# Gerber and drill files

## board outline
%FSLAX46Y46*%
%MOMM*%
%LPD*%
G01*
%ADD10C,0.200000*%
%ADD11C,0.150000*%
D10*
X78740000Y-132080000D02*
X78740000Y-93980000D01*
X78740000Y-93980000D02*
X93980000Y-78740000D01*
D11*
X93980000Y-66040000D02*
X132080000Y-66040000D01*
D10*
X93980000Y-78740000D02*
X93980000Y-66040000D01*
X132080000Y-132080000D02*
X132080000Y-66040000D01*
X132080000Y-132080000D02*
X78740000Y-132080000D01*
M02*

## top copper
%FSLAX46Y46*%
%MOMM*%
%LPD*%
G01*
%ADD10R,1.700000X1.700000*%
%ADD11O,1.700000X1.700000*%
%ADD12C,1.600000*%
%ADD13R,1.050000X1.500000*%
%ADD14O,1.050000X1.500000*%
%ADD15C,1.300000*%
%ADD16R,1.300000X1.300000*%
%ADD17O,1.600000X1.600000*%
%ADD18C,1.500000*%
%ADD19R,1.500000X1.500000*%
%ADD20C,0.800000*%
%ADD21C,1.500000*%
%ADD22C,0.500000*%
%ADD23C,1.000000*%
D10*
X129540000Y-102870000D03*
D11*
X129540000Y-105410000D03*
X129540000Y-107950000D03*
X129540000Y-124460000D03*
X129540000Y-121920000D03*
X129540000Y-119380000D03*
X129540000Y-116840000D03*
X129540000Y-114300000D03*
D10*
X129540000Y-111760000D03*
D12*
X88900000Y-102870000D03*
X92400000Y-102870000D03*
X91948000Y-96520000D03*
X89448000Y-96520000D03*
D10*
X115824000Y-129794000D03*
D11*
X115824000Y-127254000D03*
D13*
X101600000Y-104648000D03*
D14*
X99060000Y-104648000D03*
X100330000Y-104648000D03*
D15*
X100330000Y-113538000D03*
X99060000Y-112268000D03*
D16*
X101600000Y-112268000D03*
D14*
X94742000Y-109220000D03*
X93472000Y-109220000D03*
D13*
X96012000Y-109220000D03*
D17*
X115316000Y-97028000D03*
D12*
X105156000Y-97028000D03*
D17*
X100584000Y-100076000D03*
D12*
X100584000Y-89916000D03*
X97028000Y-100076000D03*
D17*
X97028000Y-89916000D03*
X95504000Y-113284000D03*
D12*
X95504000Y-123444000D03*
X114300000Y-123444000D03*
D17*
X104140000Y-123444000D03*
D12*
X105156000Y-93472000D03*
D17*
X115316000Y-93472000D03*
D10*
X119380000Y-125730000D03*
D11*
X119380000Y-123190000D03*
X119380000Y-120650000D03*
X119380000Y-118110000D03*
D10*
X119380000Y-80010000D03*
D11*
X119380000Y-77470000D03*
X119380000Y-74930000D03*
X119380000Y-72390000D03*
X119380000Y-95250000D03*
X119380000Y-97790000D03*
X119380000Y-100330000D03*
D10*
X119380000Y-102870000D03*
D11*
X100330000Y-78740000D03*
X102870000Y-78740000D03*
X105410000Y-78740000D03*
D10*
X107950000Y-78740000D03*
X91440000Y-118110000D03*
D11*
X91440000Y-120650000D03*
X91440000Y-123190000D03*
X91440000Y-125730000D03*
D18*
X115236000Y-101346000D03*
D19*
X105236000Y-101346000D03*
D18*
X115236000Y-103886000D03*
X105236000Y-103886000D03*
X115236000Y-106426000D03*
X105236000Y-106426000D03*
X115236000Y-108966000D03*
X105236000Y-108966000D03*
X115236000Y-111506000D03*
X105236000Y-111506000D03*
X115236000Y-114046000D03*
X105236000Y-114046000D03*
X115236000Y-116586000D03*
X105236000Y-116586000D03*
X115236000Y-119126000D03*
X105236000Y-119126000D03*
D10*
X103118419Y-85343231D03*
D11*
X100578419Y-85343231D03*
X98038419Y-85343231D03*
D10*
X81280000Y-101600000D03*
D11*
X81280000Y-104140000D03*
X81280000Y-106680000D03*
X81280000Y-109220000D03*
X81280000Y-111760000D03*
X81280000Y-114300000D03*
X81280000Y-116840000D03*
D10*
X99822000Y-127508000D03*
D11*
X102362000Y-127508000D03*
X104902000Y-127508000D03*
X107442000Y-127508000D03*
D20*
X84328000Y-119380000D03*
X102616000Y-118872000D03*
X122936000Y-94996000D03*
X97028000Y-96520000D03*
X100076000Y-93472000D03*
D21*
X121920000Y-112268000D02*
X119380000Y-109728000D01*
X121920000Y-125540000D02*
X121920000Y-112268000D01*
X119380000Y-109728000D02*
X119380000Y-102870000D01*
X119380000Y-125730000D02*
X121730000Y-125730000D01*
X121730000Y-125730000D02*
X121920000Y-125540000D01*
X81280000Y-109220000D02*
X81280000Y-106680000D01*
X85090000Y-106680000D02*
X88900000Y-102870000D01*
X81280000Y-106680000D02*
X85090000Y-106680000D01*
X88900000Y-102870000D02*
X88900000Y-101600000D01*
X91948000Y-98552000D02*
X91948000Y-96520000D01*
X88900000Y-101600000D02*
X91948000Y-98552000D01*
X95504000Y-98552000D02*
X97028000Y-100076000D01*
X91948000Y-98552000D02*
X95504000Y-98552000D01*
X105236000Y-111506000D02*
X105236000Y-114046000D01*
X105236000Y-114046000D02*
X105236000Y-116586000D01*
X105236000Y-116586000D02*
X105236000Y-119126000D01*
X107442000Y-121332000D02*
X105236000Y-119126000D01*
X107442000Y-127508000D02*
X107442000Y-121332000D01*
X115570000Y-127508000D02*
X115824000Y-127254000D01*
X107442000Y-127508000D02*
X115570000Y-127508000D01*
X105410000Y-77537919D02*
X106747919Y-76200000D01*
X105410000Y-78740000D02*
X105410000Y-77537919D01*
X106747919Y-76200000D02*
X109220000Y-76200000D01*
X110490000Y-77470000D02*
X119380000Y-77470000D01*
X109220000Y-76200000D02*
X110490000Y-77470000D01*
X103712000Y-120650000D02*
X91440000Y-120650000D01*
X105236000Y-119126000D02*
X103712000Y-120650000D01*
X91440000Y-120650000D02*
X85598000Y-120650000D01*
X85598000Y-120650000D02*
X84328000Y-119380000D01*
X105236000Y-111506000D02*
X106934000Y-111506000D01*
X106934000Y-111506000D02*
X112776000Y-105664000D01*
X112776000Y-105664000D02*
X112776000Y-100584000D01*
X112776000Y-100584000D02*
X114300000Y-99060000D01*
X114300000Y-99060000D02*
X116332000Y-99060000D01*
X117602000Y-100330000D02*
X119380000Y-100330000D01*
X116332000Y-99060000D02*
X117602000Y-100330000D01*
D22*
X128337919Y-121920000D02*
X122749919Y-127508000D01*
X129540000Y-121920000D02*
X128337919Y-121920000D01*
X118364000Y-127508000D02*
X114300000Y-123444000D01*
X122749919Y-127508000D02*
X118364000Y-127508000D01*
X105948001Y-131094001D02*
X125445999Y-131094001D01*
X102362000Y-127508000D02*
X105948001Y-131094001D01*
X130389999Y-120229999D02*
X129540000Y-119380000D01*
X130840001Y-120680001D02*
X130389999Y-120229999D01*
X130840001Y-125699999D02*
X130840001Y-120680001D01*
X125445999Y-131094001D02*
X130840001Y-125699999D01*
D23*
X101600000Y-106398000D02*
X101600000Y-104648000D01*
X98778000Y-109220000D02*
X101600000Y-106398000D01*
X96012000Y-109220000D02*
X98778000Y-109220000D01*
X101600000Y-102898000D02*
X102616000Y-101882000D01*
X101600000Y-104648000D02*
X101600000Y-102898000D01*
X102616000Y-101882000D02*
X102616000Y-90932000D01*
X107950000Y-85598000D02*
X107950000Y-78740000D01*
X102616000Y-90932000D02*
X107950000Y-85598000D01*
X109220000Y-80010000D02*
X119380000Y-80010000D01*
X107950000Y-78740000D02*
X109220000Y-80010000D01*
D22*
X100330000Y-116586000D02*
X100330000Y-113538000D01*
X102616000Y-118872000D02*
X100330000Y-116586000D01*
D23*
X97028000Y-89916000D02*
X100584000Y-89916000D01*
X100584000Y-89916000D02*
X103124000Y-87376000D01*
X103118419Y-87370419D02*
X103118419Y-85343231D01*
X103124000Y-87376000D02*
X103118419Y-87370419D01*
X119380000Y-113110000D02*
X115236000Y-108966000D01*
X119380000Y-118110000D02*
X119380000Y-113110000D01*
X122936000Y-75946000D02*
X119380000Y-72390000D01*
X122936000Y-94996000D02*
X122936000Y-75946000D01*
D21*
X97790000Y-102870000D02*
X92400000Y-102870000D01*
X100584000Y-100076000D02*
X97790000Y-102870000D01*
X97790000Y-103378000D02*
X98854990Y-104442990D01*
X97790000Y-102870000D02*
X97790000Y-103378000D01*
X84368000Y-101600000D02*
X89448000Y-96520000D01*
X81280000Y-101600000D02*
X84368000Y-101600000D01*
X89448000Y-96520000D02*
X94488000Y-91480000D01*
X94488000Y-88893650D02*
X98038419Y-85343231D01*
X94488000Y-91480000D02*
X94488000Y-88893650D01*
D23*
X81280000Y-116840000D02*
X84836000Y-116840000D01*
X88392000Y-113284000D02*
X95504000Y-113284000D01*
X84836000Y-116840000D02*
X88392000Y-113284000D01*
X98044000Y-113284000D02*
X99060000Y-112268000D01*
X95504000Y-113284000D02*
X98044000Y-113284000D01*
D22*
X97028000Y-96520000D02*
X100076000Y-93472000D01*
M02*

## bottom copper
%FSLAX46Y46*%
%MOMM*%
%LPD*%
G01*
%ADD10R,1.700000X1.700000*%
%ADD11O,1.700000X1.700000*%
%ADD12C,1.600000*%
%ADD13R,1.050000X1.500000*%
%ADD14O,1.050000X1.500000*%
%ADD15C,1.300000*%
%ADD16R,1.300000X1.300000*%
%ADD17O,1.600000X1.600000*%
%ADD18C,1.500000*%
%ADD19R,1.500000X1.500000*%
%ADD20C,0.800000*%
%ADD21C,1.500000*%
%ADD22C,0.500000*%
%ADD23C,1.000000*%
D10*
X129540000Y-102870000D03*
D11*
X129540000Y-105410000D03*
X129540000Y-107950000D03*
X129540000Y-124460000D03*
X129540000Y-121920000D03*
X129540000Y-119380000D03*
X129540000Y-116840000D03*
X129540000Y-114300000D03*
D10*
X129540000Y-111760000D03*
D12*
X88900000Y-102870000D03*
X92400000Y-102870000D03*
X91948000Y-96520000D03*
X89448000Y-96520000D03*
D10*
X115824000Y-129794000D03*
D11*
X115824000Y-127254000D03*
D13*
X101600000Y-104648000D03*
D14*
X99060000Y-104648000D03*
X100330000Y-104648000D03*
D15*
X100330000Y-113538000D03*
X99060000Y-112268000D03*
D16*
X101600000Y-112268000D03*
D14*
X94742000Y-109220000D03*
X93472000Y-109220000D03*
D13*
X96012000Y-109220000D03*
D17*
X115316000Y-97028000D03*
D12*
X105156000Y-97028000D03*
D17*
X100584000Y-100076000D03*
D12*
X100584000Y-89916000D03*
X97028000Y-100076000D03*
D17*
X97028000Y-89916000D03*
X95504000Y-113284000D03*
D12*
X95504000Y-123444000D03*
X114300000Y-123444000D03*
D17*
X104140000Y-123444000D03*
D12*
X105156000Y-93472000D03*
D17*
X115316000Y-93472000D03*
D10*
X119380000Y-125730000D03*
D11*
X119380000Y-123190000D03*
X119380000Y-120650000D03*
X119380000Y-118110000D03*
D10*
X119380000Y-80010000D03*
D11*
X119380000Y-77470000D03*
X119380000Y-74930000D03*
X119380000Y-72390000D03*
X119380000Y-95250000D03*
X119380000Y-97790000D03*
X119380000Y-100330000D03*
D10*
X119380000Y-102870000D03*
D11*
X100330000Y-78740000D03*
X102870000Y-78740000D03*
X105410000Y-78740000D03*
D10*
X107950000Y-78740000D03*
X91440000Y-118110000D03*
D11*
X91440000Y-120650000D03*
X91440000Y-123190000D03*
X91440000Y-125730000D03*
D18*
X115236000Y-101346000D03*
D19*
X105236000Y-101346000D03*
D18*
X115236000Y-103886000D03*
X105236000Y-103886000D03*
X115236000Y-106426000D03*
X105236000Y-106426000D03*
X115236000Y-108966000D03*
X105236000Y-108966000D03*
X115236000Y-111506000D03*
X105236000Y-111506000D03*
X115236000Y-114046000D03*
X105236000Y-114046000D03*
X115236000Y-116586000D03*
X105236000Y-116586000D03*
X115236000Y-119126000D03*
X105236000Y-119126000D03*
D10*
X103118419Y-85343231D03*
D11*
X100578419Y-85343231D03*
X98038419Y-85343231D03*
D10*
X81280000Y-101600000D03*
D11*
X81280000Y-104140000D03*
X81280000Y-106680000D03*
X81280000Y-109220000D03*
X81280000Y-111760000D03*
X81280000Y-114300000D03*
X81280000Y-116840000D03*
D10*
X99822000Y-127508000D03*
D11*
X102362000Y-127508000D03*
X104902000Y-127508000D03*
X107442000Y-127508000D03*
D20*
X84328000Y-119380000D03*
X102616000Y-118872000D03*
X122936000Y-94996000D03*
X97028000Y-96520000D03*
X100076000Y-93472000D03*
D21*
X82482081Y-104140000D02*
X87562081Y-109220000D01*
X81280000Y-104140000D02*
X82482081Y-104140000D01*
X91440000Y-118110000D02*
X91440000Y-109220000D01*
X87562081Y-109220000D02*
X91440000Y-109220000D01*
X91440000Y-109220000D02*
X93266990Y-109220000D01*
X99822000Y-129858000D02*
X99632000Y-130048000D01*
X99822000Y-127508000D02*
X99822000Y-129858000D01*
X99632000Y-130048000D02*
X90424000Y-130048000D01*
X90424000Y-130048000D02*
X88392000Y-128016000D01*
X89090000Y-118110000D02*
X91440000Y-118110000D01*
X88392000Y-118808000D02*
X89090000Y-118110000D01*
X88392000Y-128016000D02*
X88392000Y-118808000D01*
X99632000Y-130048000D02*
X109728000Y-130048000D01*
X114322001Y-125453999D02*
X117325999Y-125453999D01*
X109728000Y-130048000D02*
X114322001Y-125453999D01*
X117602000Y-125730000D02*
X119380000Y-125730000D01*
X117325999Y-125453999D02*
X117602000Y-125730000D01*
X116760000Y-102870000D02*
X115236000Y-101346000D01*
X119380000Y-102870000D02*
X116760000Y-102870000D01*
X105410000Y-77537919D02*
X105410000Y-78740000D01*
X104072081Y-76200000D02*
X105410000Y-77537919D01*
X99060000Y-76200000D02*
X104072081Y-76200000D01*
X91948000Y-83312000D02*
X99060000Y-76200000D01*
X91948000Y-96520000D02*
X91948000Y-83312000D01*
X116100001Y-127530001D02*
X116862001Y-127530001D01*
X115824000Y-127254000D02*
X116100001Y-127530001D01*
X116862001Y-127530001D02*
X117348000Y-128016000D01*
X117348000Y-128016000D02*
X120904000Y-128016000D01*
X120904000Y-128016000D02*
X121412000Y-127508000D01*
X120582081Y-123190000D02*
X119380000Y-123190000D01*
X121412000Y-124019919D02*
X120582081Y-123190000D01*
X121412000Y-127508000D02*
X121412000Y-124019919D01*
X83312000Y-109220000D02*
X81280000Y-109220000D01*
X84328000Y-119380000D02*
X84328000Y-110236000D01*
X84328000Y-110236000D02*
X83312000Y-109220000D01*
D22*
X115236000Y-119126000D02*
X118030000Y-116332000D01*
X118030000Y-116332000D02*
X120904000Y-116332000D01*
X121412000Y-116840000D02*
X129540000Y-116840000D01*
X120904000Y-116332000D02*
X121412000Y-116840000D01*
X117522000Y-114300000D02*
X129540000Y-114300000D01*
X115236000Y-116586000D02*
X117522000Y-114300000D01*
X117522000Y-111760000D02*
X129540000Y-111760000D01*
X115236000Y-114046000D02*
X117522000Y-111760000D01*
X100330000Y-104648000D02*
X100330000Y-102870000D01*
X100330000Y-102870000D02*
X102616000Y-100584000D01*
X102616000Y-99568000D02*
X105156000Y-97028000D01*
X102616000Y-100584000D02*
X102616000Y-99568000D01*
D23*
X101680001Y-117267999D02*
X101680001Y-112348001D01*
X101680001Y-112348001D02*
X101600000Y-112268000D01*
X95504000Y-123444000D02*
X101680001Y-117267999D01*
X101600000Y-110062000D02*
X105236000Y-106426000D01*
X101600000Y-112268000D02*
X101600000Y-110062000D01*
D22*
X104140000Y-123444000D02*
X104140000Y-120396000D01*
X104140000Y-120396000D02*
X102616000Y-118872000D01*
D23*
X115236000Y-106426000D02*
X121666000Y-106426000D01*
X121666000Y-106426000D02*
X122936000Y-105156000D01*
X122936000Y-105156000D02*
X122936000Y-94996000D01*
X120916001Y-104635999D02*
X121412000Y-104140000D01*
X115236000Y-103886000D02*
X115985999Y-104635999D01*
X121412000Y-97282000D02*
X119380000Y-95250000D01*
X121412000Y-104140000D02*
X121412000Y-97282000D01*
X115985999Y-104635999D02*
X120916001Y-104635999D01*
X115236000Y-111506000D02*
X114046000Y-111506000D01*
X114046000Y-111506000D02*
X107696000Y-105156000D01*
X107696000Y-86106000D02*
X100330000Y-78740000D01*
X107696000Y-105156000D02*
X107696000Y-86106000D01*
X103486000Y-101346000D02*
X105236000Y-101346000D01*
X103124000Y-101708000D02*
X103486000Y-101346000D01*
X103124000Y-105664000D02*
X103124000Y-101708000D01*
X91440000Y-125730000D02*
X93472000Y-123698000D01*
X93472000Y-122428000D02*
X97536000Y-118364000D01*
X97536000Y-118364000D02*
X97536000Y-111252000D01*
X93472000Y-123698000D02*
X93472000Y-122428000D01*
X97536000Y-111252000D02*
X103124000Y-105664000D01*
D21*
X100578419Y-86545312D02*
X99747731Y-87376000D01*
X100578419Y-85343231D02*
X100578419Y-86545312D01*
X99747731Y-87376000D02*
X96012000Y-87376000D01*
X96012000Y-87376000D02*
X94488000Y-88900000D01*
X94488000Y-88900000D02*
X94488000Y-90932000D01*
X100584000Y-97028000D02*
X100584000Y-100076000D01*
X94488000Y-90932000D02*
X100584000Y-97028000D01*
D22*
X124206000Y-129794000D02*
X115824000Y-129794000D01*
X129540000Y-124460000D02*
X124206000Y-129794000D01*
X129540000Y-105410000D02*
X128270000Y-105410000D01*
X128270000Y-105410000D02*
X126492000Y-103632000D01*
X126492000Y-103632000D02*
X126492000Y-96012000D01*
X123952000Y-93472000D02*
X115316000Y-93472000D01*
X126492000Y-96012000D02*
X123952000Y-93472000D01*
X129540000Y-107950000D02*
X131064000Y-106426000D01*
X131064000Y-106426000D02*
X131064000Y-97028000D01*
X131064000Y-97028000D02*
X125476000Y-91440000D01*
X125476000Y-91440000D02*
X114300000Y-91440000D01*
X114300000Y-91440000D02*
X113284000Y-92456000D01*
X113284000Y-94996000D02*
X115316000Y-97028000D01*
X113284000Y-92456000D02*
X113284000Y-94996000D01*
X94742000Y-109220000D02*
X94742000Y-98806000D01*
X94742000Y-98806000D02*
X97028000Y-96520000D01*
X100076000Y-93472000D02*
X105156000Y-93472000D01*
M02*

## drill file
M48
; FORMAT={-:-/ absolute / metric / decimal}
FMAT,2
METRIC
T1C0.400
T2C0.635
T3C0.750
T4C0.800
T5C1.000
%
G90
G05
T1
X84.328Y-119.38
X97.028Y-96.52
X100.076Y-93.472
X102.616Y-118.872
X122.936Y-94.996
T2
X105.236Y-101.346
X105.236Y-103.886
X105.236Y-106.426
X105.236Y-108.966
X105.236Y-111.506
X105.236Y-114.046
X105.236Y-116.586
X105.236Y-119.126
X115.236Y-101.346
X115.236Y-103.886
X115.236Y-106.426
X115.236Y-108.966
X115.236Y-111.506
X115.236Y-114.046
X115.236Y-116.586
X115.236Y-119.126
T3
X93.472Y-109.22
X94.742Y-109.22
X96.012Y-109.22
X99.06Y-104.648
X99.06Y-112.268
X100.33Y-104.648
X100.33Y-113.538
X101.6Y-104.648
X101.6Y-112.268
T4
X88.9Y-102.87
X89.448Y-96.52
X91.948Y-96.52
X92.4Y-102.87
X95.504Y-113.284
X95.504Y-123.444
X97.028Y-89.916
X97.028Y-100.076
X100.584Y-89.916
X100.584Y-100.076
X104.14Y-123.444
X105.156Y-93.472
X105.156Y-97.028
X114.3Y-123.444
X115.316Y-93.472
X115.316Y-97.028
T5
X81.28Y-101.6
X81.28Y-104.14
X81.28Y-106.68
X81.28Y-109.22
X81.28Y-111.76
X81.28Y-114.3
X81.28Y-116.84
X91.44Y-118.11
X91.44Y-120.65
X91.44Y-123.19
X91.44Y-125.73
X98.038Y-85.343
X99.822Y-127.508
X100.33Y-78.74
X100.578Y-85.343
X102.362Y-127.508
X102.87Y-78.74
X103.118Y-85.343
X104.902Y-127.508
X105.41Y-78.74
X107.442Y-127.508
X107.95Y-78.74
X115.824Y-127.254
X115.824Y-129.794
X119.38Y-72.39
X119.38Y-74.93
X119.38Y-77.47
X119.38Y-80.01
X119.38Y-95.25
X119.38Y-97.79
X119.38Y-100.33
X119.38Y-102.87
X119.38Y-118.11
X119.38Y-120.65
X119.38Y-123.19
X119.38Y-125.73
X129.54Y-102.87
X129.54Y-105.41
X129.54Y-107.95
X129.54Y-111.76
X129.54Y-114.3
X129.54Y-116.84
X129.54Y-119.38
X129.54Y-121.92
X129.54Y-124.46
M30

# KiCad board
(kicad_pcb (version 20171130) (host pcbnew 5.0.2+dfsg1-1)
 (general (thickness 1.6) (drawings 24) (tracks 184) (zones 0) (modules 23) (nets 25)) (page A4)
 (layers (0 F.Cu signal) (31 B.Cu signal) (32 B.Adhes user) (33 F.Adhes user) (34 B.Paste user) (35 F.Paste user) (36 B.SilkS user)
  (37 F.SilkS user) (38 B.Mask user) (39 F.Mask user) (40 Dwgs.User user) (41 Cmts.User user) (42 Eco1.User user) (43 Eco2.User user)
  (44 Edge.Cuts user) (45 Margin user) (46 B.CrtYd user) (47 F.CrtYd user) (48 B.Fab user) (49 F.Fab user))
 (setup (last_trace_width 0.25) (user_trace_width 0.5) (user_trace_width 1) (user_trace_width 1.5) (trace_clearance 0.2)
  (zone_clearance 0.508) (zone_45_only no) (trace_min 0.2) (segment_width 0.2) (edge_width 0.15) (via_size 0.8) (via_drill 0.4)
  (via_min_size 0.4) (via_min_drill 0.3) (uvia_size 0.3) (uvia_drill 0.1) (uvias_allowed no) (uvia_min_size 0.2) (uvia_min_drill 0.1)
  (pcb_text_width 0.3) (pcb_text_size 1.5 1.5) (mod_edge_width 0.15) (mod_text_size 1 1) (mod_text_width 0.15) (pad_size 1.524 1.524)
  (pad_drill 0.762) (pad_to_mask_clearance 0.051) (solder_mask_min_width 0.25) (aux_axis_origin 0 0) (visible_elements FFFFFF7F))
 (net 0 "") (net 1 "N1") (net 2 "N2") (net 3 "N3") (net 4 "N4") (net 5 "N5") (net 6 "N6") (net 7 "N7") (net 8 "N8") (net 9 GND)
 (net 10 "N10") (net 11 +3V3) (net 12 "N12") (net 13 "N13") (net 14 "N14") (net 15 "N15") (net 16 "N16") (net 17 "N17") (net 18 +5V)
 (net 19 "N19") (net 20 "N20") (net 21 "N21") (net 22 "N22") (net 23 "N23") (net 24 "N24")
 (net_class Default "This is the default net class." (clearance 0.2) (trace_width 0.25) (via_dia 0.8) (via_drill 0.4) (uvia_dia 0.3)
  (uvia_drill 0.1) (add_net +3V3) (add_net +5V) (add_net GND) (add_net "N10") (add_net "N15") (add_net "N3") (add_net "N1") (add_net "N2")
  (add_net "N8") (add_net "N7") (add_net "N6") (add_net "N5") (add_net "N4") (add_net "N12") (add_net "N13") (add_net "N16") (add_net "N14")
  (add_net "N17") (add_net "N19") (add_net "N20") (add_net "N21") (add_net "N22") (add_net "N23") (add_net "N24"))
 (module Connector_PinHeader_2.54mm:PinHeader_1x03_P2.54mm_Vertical (layer F.Cu) (at 129.54 102.87)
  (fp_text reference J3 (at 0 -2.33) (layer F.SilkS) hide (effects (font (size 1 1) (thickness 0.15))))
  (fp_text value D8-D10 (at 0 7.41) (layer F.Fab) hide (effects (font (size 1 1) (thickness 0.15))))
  (pad 1 thru_hole rect (at 0 0) (size 1.7 1.7) (drill 1) (layers *.Cu *.Mask))
  (pad 2 thru_hole oval (at 0 2.54) (size 1.7 1.7) (drill 1) (layers *.Cu *.Mask) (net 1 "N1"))
  (pad 3 thru_hole oval (at 0 5.08) (size 1.7 1.7) (drill 1) (layers *.Cu *.Mask) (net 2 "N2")))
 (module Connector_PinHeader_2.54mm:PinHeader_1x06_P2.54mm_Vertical (layer F.Cu) (at 129.54 111.76)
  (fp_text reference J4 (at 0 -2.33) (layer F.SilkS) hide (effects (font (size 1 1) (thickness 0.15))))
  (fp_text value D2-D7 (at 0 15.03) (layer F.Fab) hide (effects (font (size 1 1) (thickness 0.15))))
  (pad 6 thru_hole oval (at 0 12.7) (size 1.7 1.7) (drill 1) (layers *.Cu *.Mask) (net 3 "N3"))
  (pad 5 thru_hole oval (at 0 10.16) (size 1.7 1.7) (drill 1) (layers *.Cu *.Mask) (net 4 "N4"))
  (pad 4 thru_hole oval (at 0 7.62) (size 1.7 1.7) (drill 1) (layers *.Cu *.Mask) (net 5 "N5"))
  (pad 3 thru_hole oval (at 0 5.08) (size 1.7 1.7) (drill 1) (layers *.Cu *.Mask) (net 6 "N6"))
  (pad 2 thru_hole oval (at 0 2.54) (size 1.7 1.7) (drill 1) (layers *.Cu *.Mask) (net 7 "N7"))
  (pad 1 thru_hole rect (at 0 0) (size 1.7 1.7) (drill 1) (layers *.Cu *.Mask) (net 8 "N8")))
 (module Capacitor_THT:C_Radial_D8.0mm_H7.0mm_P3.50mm (layer F.Cu) (at 88.9 102.87)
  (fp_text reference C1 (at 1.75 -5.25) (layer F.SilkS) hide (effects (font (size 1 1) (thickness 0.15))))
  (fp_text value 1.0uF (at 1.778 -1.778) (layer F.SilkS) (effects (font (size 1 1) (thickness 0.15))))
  (pad 1 thru_hole circle (at 0 0) (size 1.6 1.6) (drill 0.8) (layers *.Cu *.Mask) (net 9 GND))
  (pad 2 thru_hole circle (at 3.5 0) (size 1.6 1.6) (drill 0.8) (layers *.Cu *.Mask) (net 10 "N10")))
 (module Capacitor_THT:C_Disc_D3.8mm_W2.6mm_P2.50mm (layer F.Cu) (at 91.948 96.52 180)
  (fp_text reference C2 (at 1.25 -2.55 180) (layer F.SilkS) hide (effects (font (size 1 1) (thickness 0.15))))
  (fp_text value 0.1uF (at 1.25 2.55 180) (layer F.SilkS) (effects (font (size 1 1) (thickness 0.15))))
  (pad 1 thru_hole circle (at 0 0 180) (size 1.6 1.6) (drill 0.8) (layers *.Cu *.Mask) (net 9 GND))
  (pad 2 thru_hole circle (at 2.5 0 180) (size 1.6 1.6) (drill 0.8) (layers *.Cu *.Mask) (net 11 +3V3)))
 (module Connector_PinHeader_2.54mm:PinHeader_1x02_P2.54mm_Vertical (layer F.Cu) (at 115.824 129.794 180)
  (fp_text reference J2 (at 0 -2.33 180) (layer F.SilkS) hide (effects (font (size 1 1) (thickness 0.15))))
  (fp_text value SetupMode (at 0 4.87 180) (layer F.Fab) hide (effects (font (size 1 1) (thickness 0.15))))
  (pad 1 thru_hole rect (at 0 0 180) (size 1.7 1.7) (drill 1) (layers *.Cu *.Mask) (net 3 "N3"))
  (pad 2 thru_hole oval (at 0 2.54 180) (size 1.7 1.7) (drill 1) (layers *.Cu *.Mask) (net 9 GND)))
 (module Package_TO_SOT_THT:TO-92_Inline (layer F.Cu) (at 101.6 104.648 180)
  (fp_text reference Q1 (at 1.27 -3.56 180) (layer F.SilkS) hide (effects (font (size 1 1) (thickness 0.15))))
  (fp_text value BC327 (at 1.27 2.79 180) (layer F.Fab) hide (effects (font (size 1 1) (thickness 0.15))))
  (pad 1 thru_hole rect (at 0 0 180) (size 1.05 1.5) (drill 0.75) (layers *.Cu *.Mask) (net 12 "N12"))
  (pad 3 thru_hole oval (at 2.54 0 180) (size 1.05 1.5) (drill 0.75) (layers *.Cu *.Mask) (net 10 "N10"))
  (pad 2 thru_hole oval (at 1.27 0 180) (size 1.05 1.5) (drill 0.75) (layers *.Cu *.Mask) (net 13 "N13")))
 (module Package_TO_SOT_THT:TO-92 (layer F.Cu) (at 101.6 112.268 180)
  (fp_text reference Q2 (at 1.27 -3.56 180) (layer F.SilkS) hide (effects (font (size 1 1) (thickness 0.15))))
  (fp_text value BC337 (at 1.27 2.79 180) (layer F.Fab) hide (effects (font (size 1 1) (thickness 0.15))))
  (pad 2 thru_hole circle (at 1.27 -1.27 270) (size 1.3 1.3) (drill 0.75) (layers *.Cu *.Mask) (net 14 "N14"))
  (pad 3 thru_hole circle (at 2.54 0 270) (size 1.3 1.3) (drill 0.75) (layers *.Cu *.Mask) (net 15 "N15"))
  (pad 1 thru_hole rect (at 0 0 270) (size 1.3 1.3) (drill 0.75) (layers *.Cu *.Mask) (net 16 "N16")))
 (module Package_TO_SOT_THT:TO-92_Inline (layer F.Cu) (at 96.012 109.22 180)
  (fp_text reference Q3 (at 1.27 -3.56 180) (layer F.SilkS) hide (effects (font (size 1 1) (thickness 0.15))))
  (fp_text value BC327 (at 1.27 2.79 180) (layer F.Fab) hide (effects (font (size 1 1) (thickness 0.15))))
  (pad 2 thru_hole oval (at 1.27 0 180) (size 1.05 1.5) (drill 0.75) (layers *.Cu *.Mask) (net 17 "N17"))
  (pad 3 thru_hole oval (at 2.54 0 180) (size 1.05 1.5) (drill 0.75) (layers *.Cu *.Mask) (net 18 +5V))
  (pad 1 thru_hole rect (at 0 0 180) (size 1.05 1.5) (drill 0.75) (layers *.Cu *.Mask) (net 12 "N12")))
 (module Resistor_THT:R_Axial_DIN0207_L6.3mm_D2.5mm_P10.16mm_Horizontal (layer F.Cu) (at 105.156 97.028)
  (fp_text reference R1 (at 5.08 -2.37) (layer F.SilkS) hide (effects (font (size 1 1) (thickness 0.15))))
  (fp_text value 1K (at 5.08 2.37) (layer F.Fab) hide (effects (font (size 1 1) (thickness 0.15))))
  (pad 2 thru_hole oval (at 10.16 0) (size 1.6 1.6) (drill 0.8) (layers *.Cu *.Mask) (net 2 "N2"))
  (pad 1 thru_hole circle (at 0 0) (size 1.6 1.6) (drill 0.8) (layers *.Cu *.Mask) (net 13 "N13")))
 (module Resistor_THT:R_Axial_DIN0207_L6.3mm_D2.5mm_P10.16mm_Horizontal (layer F.Cu) (at 100.584 89.916 270)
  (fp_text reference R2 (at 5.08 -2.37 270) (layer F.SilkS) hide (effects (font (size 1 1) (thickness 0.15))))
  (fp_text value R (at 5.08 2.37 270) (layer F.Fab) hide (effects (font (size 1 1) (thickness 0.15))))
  (pad 2 thru_hole oval (at 10.16 0 270) (size 1.6 1.6) (drill 0.8) (layers *.Cu *.Mask) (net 10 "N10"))
  (pad 1 thru_hole circle (at 0 0 270) (size 1.6 1.6) (drill 0.8) (layers *.Cu *.Mask) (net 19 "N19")))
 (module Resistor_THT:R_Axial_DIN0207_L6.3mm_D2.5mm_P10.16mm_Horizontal (layer F.Cu) (at 97.028 100.076 90)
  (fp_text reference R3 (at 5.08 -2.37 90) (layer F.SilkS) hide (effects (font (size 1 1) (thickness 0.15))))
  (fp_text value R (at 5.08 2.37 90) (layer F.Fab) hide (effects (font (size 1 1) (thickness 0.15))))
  (pad 1 thru_hole circle (at 0 0 90) (size 1.6 1.6) (drill 0.8) (layers *.Cu *.Mask) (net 9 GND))
  (pad 2 thru_hole oval (at 10.16 0 90) (size 1.6 1.6) (drill 0.8) (layers *.Cu *.Mask) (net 19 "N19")))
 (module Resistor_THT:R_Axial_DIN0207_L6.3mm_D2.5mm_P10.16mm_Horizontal (layer F.Cu) (at 95.504 123.444 90)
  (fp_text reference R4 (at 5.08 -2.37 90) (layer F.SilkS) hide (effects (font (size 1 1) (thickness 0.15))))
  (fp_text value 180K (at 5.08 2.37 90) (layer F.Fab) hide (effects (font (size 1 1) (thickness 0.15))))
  (pad 2 thru_hole oval (at 10.16 0 90) (size 1.6 1.6) (drill 0.8) (layers *.Cu *.Mask) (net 15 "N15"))
  (pad 1 thru_hole circle (at 0 0 90) (size 1.6 1.6) (drill 0.8) (layers *.Cu *.Mask) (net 16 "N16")))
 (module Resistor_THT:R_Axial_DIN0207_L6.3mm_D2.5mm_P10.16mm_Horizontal (layer F.Cu) (at 114.3 123.444 180)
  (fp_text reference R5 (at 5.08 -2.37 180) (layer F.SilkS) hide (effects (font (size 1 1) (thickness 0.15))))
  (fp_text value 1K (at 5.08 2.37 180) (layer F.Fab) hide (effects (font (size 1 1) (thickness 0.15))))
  (pad 1 thru_hole circle (at 0 0 180) (size 1.6 1.6) (drill 0.8) (layers *.Cu *.Mask) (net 4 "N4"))
  (pad 2 thru_hole oval (at 10.16 0 180) (size 1.6 1.6) (drill 0.8) (layers *.Cu *.Mask) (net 14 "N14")))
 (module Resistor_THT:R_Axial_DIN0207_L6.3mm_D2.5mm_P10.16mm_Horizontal (layer F.Cu) (at 105.156 93.472)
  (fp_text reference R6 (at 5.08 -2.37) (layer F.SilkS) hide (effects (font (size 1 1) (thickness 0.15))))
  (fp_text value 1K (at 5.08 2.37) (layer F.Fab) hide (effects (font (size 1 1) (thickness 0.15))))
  (pad 1 thru_hole circle (at 0 0) (size 1.6 1.6) (drill 0.8) (layers *.Cu *.Mask) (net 17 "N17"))
  (pad 2 thru_hole oval (at 10.16 0) (size 1.6 1.6) (drill 0.8) (layers *.Cu *.Mask) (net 1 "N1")))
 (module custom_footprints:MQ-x (layer F.Cu) (at 119.38 121.92 180)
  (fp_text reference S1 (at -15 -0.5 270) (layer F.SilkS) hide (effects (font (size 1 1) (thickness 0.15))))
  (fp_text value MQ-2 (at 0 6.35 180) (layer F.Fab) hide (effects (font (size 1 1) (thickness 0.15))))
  (pad 1 thru_hole rect (at 0 -3.81 180) (size 1.7 1.7) (drill 1) (layers *.Cu *.Mask) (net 18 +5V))
  (pad 2 thru_hole oval (at 0 -1.27 180) (size 1.7 1.7) (drill 1) (layers *.Cu *.Mask) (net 9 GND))
  (pad 3 thru_hole oval (at 0 1.27 180) (size 1.7 1.7) (drill 1) (layers *.Cu *.Mask))
  (pad 4 thru_hole oval (at 0 3.81 180) (size 1.7 1.7) (drill 1) (layers *.Cu *.Mask) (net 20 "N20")))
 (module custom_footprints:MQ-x (layer F.Cu) (at 119.38 76.2 180)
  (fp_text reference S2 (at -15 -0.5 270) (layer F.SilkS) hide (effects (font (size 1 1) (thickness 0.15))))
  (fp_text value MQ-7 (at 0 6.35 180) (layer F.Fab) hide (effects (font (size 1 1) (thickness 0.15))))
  (pad 1 thru_hole rect (at 0 -3.81 180) (size 1.7 1.7) (drill 1) (layers *.Cu *.Mask) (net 12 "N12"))
  (pad 2 thru_hole oval (at 0 -1.27 180) (size 1.7 1.7) (drill 1) (layers *.Cu *.Mask) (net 9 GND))
  (pad 3 thru_hole oval (at 0 1.27 180) (size 1.7 1.7) (drill 1) (layers *.Cu *.Mask))
  (pad 4 thru_hole oval (at 0 3.81 180) (size 1.7 1.7) (drill 1) (layers *.Cu *.Mask) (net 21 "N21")))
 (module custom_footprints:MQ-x (layer F.Cu) (at 119.38 99.06 180)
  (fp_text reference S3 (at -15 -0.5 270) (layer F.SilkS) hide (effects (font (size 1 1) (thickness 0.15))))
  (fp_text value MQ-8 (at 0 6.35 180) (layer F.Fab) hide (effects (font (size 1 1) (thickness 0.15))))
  (pad 4 thru_hole oval (at 0 3.81 180) (size 1.7 1.7) (drill 1) (layers *.Cu *.Mask) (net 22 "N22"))
  (pad 3 thru_hole oval (at 0 1.27 180) (size 1.7 1.7) (drill 1) (layers *.Cu *.Mask))
  (pad 2 thru_hole oval (at 0 -1.27 180) (size 1.7 1.7) (drill 1) (layers *.Cu *.Mask) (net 9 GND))
  (pad 1 thru_hole rect (at 0 -3.81 180) (size 1.7 1.7) (drill 1) (layers *.Cu *.Mask) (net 18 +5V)))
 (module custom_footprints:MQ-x (layer F.Cu) (at 104.14 78.74 270)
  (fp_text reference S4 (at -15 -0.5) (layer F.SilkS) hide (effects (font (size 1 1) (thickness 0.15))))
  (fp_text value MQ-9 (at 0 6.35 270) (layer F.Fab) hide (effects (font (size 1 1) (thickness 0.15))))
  (pad 4 thru_hole oval (at 0 3.81 270) (size 1.7 1.7) (drill 1) (layers *.Cu *.Mask) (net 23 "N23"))
  (pad 3 thru_hole oval (at 0 1.27 270) (size 1.7 1.7) (drill 1) (layers *.Cu *.Mask))
  (pad 2 thru_hole oval (at 0 -1.27 270) (size 1.7 1.7) (drill 1) (layers *.Cu *.Mask) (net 9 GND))
  (pad 1 thru_hole rect (at 0 -3.81 270) (size 1.7 1.7) (drill 1) (layers *.Cu *.Mask) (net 12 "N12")))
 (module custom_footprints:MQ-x (layer F.Cu) (at 91.44 121.92)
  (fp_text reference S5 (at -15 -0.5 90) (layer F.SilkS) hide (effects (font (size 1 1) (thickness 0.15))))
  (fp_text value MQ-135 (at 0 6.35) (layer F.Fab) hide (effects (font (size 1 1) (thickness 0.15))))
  (pad 1 thru_hole rect (at 0 -3.81) (size 1.7 1.7) (drill 1) (layers *.Cu *.Mask) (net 18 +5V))
  (pad 2 thru_hole oval (at 0 -1.27) (size 1.7 1.7) (drill 1) (layers *.Cu *.Mask) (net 9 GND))
  (pad 3 thru_hole oval (at 0 1.27) (size 1.7 1.7) (drill 1) (layers *.Cu *.Mask))
  (pad 4 thru_hole oval (at 0 3.81) (size 1.7 1.7) (drill 1) (layers *.Cu *.Mask) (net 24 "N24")))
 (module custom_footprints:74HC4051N (layer F.Cu) (at 110.236 110.236 270)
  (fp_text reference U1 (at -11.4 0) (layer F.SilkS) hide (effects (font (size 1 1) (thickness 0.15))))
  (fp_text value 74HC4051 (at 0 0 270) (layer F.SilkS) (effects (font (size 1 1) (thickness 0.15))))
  (pad 16 thru_hole circle (at -8.89 -5 270) (size 1.5 1.5) (drill 0.635) (layers *.Cu *.Mask) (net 18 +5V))
  (pad 1 thru_hole rect (at -8.89 5 270) (size 1.5 1.5) (drill 0.635) (layers *.Cu *.Mask) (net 24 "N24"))
  (pad 15 thru_hole circle (at -6.35 -5 270) (size 1.5 1.5) (drill 0.635) (layers *.Cu *.Mask) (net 22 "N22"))
  (pad 2 thru_hole circle (at -6.35 5 270) (size 1.5 1.5) (drill 0.635) (layers *.Cu *.Mask))
  (pad 14 thru_hole circle (at -3.81 -5 270) (size 1.5 1.5) (drill 0.635) (layers *.Cu *.Mask) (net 21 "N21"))
  (pad 3 thru_hole circle (at -3.81 5 270) (size 1.5 1.5) (drill 0.635) (layers *.Cu *.Mask) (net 16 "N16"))
  (pad 13 thru_hole circle (at -1.27 -5 270) (size 1.5 1.5) (drill 0.635) (layers *.Cu *.Mask) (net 20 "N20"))
  (pad 4 thru_hole circle (at -1.27 5 270) (size 1.5 1.5) (drill 0.635) (layers *.Cu *.Mask))
  (pad 12 thru_hole circle (at 1.27 -5 270) (size 1.5 1.5) (drill 0.635) (layers *.Cu *.Mask) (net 23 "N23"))
  (pad 5 thru_hole circle (at 1.27 5 270) (size 1.5 1.5) (drill 0.635) (layers *.Cu *.Mask) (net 9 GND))
  (pad 11 thru_hole circle (at 3.81 -5 270) (size 1.5 1.5) (drill 0.635) (layers *.Cu *.Mask) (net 8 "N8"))
  (pad 6 thru_hole circle (at 3.81 5 270) (size 1.5 1.5) (drill 0.635) (layers *.Cu *.Mask) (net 9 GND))
  (pad 10 thru_hole circle (at 6.35 -5 270) (size 1.5 1.5) (drill 0.635) (layers *.Cu *.Mask) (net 7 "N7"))
  (pad 7 thru_hole circle (at 6.35 5 270) (size 1.5 1.5) (drill 0.635) (layers *.Cu *.Mask) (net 9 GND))
  (pad 9 thru_hole circle (at 8.89 -5 270) (size 1.5 1.5) (drill 0.635) (layers *.Cu *.Mask) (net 6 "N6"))
  (pad 8 thru_hole circle (at 8.89 5 270) (size 1.5 1.5) (drill 0.635) (layers *.Cu *.Mask) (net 9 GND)))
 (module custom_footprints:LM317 (layer F.Cu) (at 100.584 85.344 180)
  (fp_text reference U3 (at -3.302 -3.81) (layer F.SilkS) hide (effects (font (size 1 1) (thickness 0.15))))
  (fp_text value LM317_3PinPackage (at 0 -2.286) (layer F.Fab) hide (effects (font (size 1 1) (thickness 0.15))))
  (pad 1 thru_hole rect (at -2.534419 0.000769 270) (size 1.7 1.7) (drill 1) (layers *.Cu *.Mask) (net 19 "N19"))
  (pad 2 thru_hole oval (at 0.005581 0.000769) (size 1.7 1.7) (drill 1) (layers *.Cu *.Mask) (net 10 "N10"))
  (pad 3 thru_hole oval (at 2.545581 0.000769 270) (size 1.7 1.7) (drill 1) (layers *.Cu *.Mask) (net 11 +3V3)))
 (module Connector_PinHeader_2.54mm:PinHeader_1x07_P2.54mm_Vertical (layer F.Cu) (at 81.28 101.6)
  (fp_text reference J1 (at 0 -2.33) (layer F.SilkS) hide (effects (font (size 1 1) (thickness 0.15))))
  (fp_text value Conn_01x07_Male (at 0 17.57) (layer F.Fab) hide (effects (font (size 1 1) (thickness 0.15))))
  (pad 1 thru_hole rect (at 0 0) (size 1.7 1.7) (drill 1) (layers *.Cu *.Mask) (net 11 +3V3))
  (pad 2 thru_hole oval (at 0 2.54) (size 1.7 1.7) (drill 1) (layers *.Cu *.Mask) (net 18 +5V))
  (pad 3 thru_hole oval (at 0 5.08) (size 1.7 1.7) (drill 1) (layers *.Cu *.Mask) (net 9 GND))
  (pad 4 thru_hole oval (at 0 7.62) (size 1.7 1.7) (drill 1) (layers *.Cu *.Mask) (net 9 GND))
  (pad 5 thru_hole oval (at 0 10.16) (size 1.7 1.7) (drill 1) (layers *.Cu *.Mask))
  (pad 6 thru_hole oval (at 0 12.7) (size 1.7 1.7) (drill 1) (layers *.Cu *.Mask))
  (pad 7 thru_hole oval (at 0 15.24) (size 1.7 1.7) (drill 1) (layers *.Cu *.Mask) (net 15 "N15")))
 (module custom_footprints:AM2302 (layer F.Cu) (at 103.632 127.508)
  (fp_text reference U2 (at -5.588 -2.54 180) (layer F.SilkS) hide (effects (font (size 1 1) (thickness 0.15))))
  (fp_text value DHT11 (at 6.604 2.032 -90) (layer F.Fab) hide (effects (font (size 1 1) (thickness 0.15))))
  (pad 1 thru_hole rect (at -3.81 0 90) (size 1.7 1.7) (drill 1) (layers *.Cu *.Mask) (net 18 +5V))
  (pad 2 thru_hole oval (at -1.27 0 90) (size 1.7 1.7) (drill 1) (layers *.Cu *.Mask) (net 5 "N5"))
  (pad 3 thru_hole oval (at 1.27 0 90) (size 1.7 1.7) (drill 1) (layers *.Cu *.Mask))
  (pad 4 thru_hole oval (at 3.81 0 90) (size 1.7 1.7) (drill 1) (layers *.Cu *.Mask) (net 9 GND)))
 (gr_line (start 78.74 132.08) (end 78.74 93.98) (layer Edge.Cuts) (width 0.2))
 (gr_line (start 78.74 93.98) (end 93.98 78.74) (layer Edge.Cuts) (width 0.2))
 (gr_line (start 93.98 66.04) (end 132.08 66.04) (layer Edge.Cuts) (width 0.15))
 (gr_line (start 93.98 78.74) (end 93.98 66.04) (layer Edge.Cuts) (width 0.2))
 (gr_line (start 132.08 132.08) (end 132.08 66.04) (layer Edge.Cuts) (width 0.2))
 (gr_line (start 132.08 132.08) (end 78.74 132.08) (layer Edge.Cuts) (width 0.2))
 (segment (start 82.482081 104.14) (end 87.562081 109.22) (width 1.5) (layer B.Cu) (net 18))
 (segment (start 81.28 104.14) (end 82.482081 104.14) (width 1.5) (layer B.Cu) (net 18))
 (segment (start 91.44 118.11) (end 91.44 109.22) (width 1.5) (layer B.Cu) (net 18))
 (segment (start 87.562081 109.22) (end 91.44 109.22) (width 1.5) (layer B.Cu) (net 18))
 (segment (start 91.44 109.22) (end 93.26699 109.22) (width 1.5) (layer B.Cu) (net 18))
 (segment (start 99.822 129.858) (end 99.632 130.048) (width 1.5) (layer B.Cu) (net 18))
 (segment (start 99.822 127.508) (end 99.822 129.858) (width 1.5) (layer B.Cu) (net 18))
 (segment (start 99.632 130.048) (end 90.424 130.048) (width 1.5) (layer B.Cu) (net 18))
 (segment (start 90.424 130.048) (end 88.392 128.016) (width 1.5) (layer B.Cu) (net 18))
 (segment (start 89.09 118.11) (end 91.44 118.11) (width 1.5) (layer B.Cu) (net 18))
 (segment (start 88.392 118.808) (end 89.09 118.11) (width 1.5) (layer B.Cu) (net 18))
 (segment (start 88.392 128.016) (end 88.392 118.808) (width 1.5) (layer B.Cu) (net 18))
 (segment (start 99.632 130.048) (end 109.728 130.048) (width 1.5) (layer B.Cu) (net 18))
 (segment (start 114.322001 125.453999) (end 117.325999 125.453999) (width 1.5) (layer B.Cu) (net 18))
 (segment (start 109.728 130.048) (end 114.322001 125.453999) (width 1.5) (layer B.Cu) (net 18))
 (segment (start 117.602 125.73) (end 119.38 125.73) (width 1.5) (layer B.Cu) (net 18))
 (segment (start 117.325999 125.453999) (end 117.602 125.73) (width 1.5) (layer B.Cu) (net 18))
 (segment (start 116.76 102.87) (end 115.236 101.346) (width 1.5) (layer B.Cu) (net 18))
 (segment (start 119.38 102.87) (end 116.76 102.87) (width 1.5) (layer B.Cu) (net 18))
 (segment (start 121.92 112.268) (end 119.38 109.728) (width 1.5) (layer F.Cu) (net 18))
 (segment (start 121.92 125.54) (end 121.92 112.268) (width 1.5) (layer F.Cu) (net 18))
 (segment (start 119.38 109.728) (end 119.38 102.87) (width 1.5) (layer F.Cu) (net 18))
 (segment (start 119.38 125.73) (end 121.73 125.73) (width 1.5) (layer F.Cu) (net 18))
 (segment (start 121.73 125.73) (end 121.92 125.54) (width 1.5) (layer F.Cu) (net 18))
 (segment (start 81.28 109.22) (end 81.28 106.68) (width 1.5) (layer F.Cu) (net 9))
 (segment (start 85.09 106.68) (end 88.9 102.87) (width 1.5) (layer F.Cu) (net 9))
 (segment (start 81.28 106.68) (end 85.09 106.68) (width 1.5) (layer F.Cu) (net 9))
 (segment (start 88.9 102.87) (end 88.9 101.6) (width 1.5) (layer F.Cu) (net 9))
 (segment (start 91.948 98.552) (end 91.948 96.52) (width 1.5) (layer F.Cu) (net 9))
 (segment (start 88.9 101.6) (end 91.948 98.552) (width 1.5) (layer F.Cu) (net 9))
 (segment (start 95.504 98.552) (end 97.028 100.076) (width 1.5) (layer F.Cu) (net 9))
 (segment (start 91.948 98.552) (end 95.504 98.552) (width 1.5) (layer F.Cu) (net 9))
 (segment (start 105.236 111.506) (end 105.236 114.046) (width 1.5) (layer F.Cu) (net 9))
 (segment (start 105.236 114.046) (end 105.236 116.586) (width 1.5) (layer F.Cu) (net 9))
 (segment (start 105.236 116.586) (end 105.236 119.126) (width 1.5) (layer F.Cu) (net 9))
 (segment (start 107.442 121.332) (end 105.236 119.126) (width 1.5) (layer F.Cu) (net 9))
 (segment (start 107.442 127.508) (end 107.442 121.332) (width 1.5) (layer F.Cu) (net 9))
 (segment (start 115.57 127.508) (end 115.824 127.254) (width 1.5) (layer F.Cu) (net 9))
 (segment (start 107.442 127.508) (end 115.57 127.508) (width 1.5) (layer F.Cu) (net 9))
 (segment (start 105.41 77.537919) (end 106.747919 76.2) (width 1.5) (layer F.Cu) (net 9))
 (segment (start 105.41 78.74) (end 105.41 77.537919) (width 1.5) (layer F.Cu) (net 9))
 (segment (start 106.747919 76.2) (end 109.22 76.2) (width 1.5) (layer F.Cu) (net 9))
 (segment (start 110.49 77.47) (end 119.38 77.47) (width 1.5) (layer F.Cu) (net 9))
 (segment (start 109.22 76.2) (end 110.49 77.47) (width 1.5) (layer F.Cu) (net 9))
 (segment (start 105.41 77.537919) (end 105.41 78.74) (width 1.5) (layer B.Cu) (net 9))
 (segment (start 104.072081 76.2) (end 105.41 77.537919) (width 1.5) (layer B.Cu) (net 9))
 (segment (start 99.06 76.2) (end 104.072081 76.2) (width 1.5) (layer B.Cu) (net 9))
 (segment (start 91.948 83.312) (end 99.06 76.2) (width 1.5) (layer B.Cu) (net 9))
 (segment (start 91.948 96.52) (end 91.948 83.312) (width 1.5) (layer B.Cu) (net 9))
 (segment (start 116.100001 127.530001) (end 116.862001 127.530001) (width 1.5) (layer B.Cu) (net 9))
 (segment (start 115.824 127.254) (end 116.100001 127.530001) (width 1.5) (layer B.Cu) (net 9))
 (segment (start 116.862001 127.530001) (end 117.348 128.016) (width 1.5) (layer B.Cu) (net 9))
 (segment (start 117.348 128.016) (end 120.904 128.016) (width 1.5) (layer B.Cu) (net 9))
 (segment (start 120.904 128.016) (end 121.412 127.508) (width 1.5) (layer B.Cu) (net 9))
 (segment (start 120.582081 123.19) (end 119.38 123.19) (width 1.5) (layer B.Cu) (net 9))
 (segment (start 121.412 124.019919) (end 120.582081 123.19) (width 1.5) (layer B.Cu) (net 9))
 (segment (start 121.412 127.508) (end 121.412 124.019919) (width 1.5) (layer B.Cu) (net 9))
 (segment (start 103.712 120.65) (end 91.44 120.65) (width 1.5) (layer F.Cu) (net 9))
 (segment (start 105.236 119.126) (end 103.712 120.65) (width 1.5) (layer F.Cu) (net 9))
 (segment (start 91.44 120.65) (end 85.598 120.65) (width 1.5) (layer F.Cu) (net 9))
 (segment (start 85.598 120.65) (end 84.328 119.38) (width 1.5) (layer F.Cu) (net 9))
 (via (at 84.328 119.38) (size 0.8) (drill 0.4) (layers F.Cu B.Cu) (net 9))
 (segment (start 83.312 109.22) (end 81.28 109.22) (width 1.5) (layer B.Cu) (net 9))
 (segment (start 84.328 119.38) (end 84.328 110.236) (width 1.5) (layer B.Cu) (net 9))
 (segment (start 84.328 110.236) (end 83.312 109.22) (width 1.5) (layer B.Cu) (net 9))
 (segment (start 105.236 111.506) (end 106.934 111.506) (width 1.5) (layer F.Cu) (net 9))
 (segment (start 106.934 111.506) (end 112.776 105.664) (width 1.5) (layer F.Cu) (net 9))
 (segment (start 112.776 105.664) (end 112.776 100.584) (width 1.5) (layer F.Cu) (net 9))
 (segment (start 112.776 100.584) (end 114.3 99.06) (width 1.5) (layer F.Cu) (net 9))
 (segment (start 114.3 99.06) (end 116.332 99.06) (width 1.5) (layer F.Cu) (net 9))
 (segment (start 117.602 100.33) (end 119.38 100.33) (width 1.5) (layer F.Cu) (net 9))
 (segment (start 116.332 99.06) (end 117.602 100.33) (width 1.5) (layer F.Cu) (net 9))
 (segment (start 128.337919 121.92) (end 122.749919 127.508) (width 0.5) (layer F.Cu) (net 4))
 (segment (start 129.54 121.92) (end 128.337919 121.92) (width 0.5) (layer F.Cu) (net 4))
 (segment (start 118.364 127.508) (end 114.3 123.444) (width 0.5) (layer F.Cu) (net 4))
 (segment (start 122.749919 127.508) (end 118.364 127.508) (width 0.5) (layer F.Cu) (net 4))
 (segment (start 105.948001 131.094001) (end 125.445999 131.094001) (width 0.5) (layer F.Cu) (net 5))
 (segment (start 102.362 127.508) (end 105.948001 131.094001) (width 0.5) (layer F.Cu) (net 5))
 (segment (start 130.389999 120.229999) (end 129.54 119.38) (width 0.5) (layer F.Cu) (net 5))
 (segment (start 130.840001 120.680001) (end 130.389999 120.229999) (width 0.5) (layer F.Cu) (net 5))
 (segment (start 130.840001 125.699999) (end 130.840001 120.680001) (width 0.5) (layer F.Cu) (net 5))
 (segment (start 125.445999 131.094001) (end 130.840001 125.699999) (width 0.5) (layer F.Cu) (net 5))
 (segment (start 115.236 119.126) (end 118.03 116.332) (width 0.5) (layer B.Cu) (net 6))
 (segment (start 118.03 116.332) (end 120.904 116.332) (width 0.5) (layer B.Cu) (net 6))
 (segment (start 121.412 116.84) (end 129.54 116.84) (width 0.5) (layer B.Cu) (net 6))
 (segment (start 120.904 116.332) (end 121.412 116.84) (width 0.5) (layer B.Cu) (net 6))
 (segment (start 117.522 114.3) (end 129.54 114.3) (width 0.5) (layer B.Cu) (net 7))
 (segment (start 115.236 116.586) (end 117.522 114.3) (width 0.5) (layer B.Cu) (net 7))
 (segment (start 117.522 111.76) (end 129.54 111.76) (width 0.5) (layer B.Cu) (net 8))
 (segment (start 115.236 114.046) (end 117.522 111.76) (width 0.5) (layer B.Cu) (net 8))
 (segment (start 100.33 104.648) (end 100.33 102.87) (width 0.5) (layer B.Cu) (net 13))
 (segment (start 100.33 102.87) (end 102.616 100.584) (width 0.5) (layer B.Cu) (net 13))
 (segment (start 102.616 99.568) (end 105.156 97.028) (width 0.5) (layer B.Cu) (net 13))
 (segment (start 102.616 100.584) (end 102.616 99.568) (width 0.5) (layer B.Cu) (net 13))
 (segment (start 101.6 106.398) (end 101.6 104.648) (width 1) (layer F.Cu) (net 12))
 (segment (start 98.778 109.22) (end 101.6 106.398) (width 1) (layer F.Cu) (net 12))
 (segment (start 96.012 109.22) (end 98.778 109.22) (width 1) (layer F.Cu) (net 12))
 (segment (start 101.6 102.898) (end 102.616 101.882) (width 1) (layer F.Cu) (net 12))
 (segment (start 101.6 104.648) (end 101.6 102.898) (width 1) (layer F.Cu) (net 12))
 (segment (start 102.616 101.882) (end 102.616 90.932) (width 1) (layer F.Cu) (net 12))
 (segment (start 107.95 85.598) (end 107.95 78.74) (width 1) (layer F.Cu) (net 12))
 (segment (start 102.616 90.932) (end 107.95 85.598) (width 1) (layer F.Cu) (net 12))
 (segment (start 109.22 80.01) (end 119.38 80.01) (width 1) (layer F.Cu) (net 12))
 (segment (start 107.95 78.74) (end 109.22 80.01) (width 1) (layer F.Cu) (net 12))
 (segment (start 101.680001 117.267999) (end 101.680001 112.348001) (width 1) (layer B.Cu) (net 16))
 (segment (start 101.680001 112.348001) (end 101.6 112.268) (width 1) (layer B.Cu) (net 16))
 (segment (start 95.504 123.444) (end 101.680001 117.267999) (width 1) (layer B.Cu) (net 16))
 (segment (start 101.6 110.062) (end 105.236 106.426) (width 1) (layer B.Cu) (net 16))
 (segment (start 101.6 112.268) (end 101.6 110.062) (width 1) (layer B.Cu) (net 16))
 (segment (start 104.14 123.444) (end 104.14 120.396) (width 0.5) (layer B.Cu) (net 14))
 (segment (start 104.14 120.396) (end 102.616 118.872) (width 0.5) (layer B.Cu) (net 14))
 (via (at 102.616 118.872) (size 0.8) (drill 0.4) (layers F.Cu B.Cu) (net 14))
 (segment (start 100.33 116.586) (end 100.33 113.538) (width 0.5) (layer F.Cu) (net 14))
 (segment (start 102.616 118.872) (end 100.33 116.586) (width 0.5) (layer F.Cu) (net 14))
 (segment (start 97.028 89.916) (end 100.584 89.916) (width 1) (layer F.Cu) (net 19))
 (segment (start 100.584 89.916) (end 103.124 87.376) (width 1) (layer F.Cu) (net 19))
 (segment (start 103.118419 87.370419) (end 103.118419 85.343231) (width 1) (layer F.Cu) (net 19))
 (segment (start 103.124 87.376) (end 103.118419 87.370419) (width 1) (layer F.Cu) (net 19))
 (segment (start 119.38 113.11) (end 115.236 108.966) (width 1) (layer F.Cu) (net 20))
 (segment (start 119.38 118.11) (end 119.38 113.11) (width 1) (layer F.Cu) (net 20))
 (segment (start 115.236 106.426) (end 121.666 106.426) (width 1) (layer B.Cu) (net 21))
 (segment (start 121.666 106.426) (end 122.936 105.156) (width 1) (layer B.Cu) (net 21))
 (segment (start 122.936 105.156) (end 122.936 94.996) (width 1) (layer B.Cu) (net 21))
 (via (at 122.936 94.996) (size 0.8) (drill 0.4) (layers F.Cu B.Cu) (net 21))
 (segment (start 122.936 75.946) (end 119.38 72.39) (width 1) (layer F.Cu) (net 21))
 (segment (start 122.936 94.996) (end 122.936 75.946) (width 1) (layer F.Cu) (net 21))
 (segment (start 120.916001 104.635999) (end 121.412 104.14) (width 1) (layer B.Cu) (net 22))
 (segment (start 115.236 103.886) (end 115.985999 104.635999) (width 1) (layer B.Cu) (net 22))
 (segment (start 121.412 97.282) (end 119.38 95.25) (width 1) (layer B.Cu) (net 22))
 (segment (start 121.412 104.14) (end 121.412 97.282) (width 1) (layer B.Cu) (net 22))
 (segment (start 115.985999 104.635999) (end 120.916001 104.635999) (width 1) (layer B.Cu) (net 22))
 (segment (start 115.236 111.506) (end 114.046 111.506) (width 1) (layer B.Cu) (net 23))
 (segment (start 114.046 111.506) (end 107.696 105.156) (width 1) (layer B.Cu) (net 23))
 (segment (start 107.696 86.106) (end 100.33 78.74) (width 1) (layer B.Cu) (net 23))
 (segment (start 107.696 105.156) (end 107.696 86.106) (width 1) (layer B.Cu) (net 23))
 (segment (start 103.486 101.346) (end 105.236 101.346) (width 1) (layer B.Cu) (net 24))
 (segment (start 103.124 101.708) (end 103.486 101.346) (width 1) (layer B.Cu) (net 24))
 (segment (start 103.124 105.664) (end 103.124 101.708) (width 1) (layer B.Cu) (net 24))
 (segment (start 91.44 125.73) (end 93.472 123.698) (width 1) (layer B.Cu) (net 24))
 (segment (start 93.472 122.428) (end 97.536 118.364) (width 1) (layer B.Cu) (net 24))
 (segment (start 97.536 118.364) (end 97.536 111.252) (width 1) (layer B.Cu) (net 24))
 (segment (start 93.472 123.698) (end 93.472 122.428) (width 1) (layer B.Cu) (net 24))
 (segment (start 97.536 111.252) (end 103.124 105.664) (width 1) (layer B.Cu) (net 24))
 (segment (start 100.578419 86.545312) (end 99.747731 87.376) (width 1.5) (layer B.Cu) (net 10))
 (segment (start 100.578419 85.343231) (end 100.578419 86.545312) (width 1.5) (layer B.Cu) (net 10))
 (segment (start 99.747731 87.376) (end 96.012 87.376) (width 1.5) (layer B.Cu) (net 10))
 (segment (start 96.012 87.376) (end 94.488 88.9) (width 1.5) (layer B.Cu) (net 10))
 (segment (start 94.488 88.9) (end 94.488 90.932) (width 1.5) (layer B.Cu) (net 10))
 (segment (start 100.584 97.028) (end 100.584 100.076) (width 1.5) (layer B.Cu) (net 10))
 (segment (start 94.488 90.932) (end 100.584 97.028) (width 1.5) (layer B.Cu) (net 10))
 (segment (start 97.79 102.87) (end 92.4 102.87) (width 1.5) (layer F.Cu) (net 10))
 (segment (start 100.584 100.076) (end 97.79 102.87) (width 1.5) (layer F.Cu) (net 10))
 (segment (start 97.79 103.378) (end 98.85499 104.44299) (width 1.5) (layer F.Cu) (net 10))
 (segment (start 97.79 102.87) (end 97.79 103.378) (width 1.5) (layer F.Cu) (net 10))
 (segment (start 84.368 101.6) (end 89.448 96.52) (width 1.5) (layer F.Cu) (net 11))
 (segment (start 81.28 101.6) (end 84.368 101.6) (width 1.5) (layer F.Cu) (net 11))
 (segment (start 89.448 96.52) (end 94.488 91.48) (width 1.5) (layer F.Cu) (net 11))
 (segment (start 94.488 88.89365) (end 98.038419 85.343231) (width 1.5) (layer F.Cu) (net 11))
 (segment (start 94.488 91.48) (end 94.488 88.89365) (width 1.5) (layer F.Cu) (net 11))
 (segment (start 81.28 116.84) (end 84.836 116.84) (width 1) (layer F.Cu) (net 15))
 (segment (start 88.392 113.284) (end 95.504 113.284) (width 1) (layer F.Cu) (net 15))
 (segment (start 84.836 116.84) (end 88.392 113.284) (width 1) (layer F.Cu) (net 15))
 (segment (start 98.044 113.284) (end 99.06 112.268) (width 1) (layer F.Cu) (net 15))
 (segment (start 95.504 113.284) (end 98.044 113.284) (width 1) (layer F.Cu) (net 15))
 (segment (start 124.206 129.794) (end 115.824 129.794) (width 0.5) (layer B.Cu) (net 3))
 (segment (start 129.54 124.46) (end 124.206 129.794) (width 0.5) (layer B.Cu) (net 3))
 (segment (start 129.54 105.41) (end 128.27 105.41) (width 0.5) (layer B.Cu) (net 1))
 (segment (start 128.27 105.41) (end 126.492 103.632) (width 0.5) (layer B.Cu) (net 1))
 (segment (start 126.492 103.632) (end 126.492 96.012) (width 0.5) (layer B.Cu) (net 1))
 (segment (start 123.952 93.472) (end 115.316 93.472) (width 0.5) (layer B.Cu) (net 1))
 (segment (start 126.492 96.012) (end 123.952 93.472) (width 0.5) (layer B.Cu) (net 1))
 (segment (start 129.54 107.95) (end 131.064 106.426) (width 0.5) (layer B.Cu) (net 2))
 (segment (start 131.064 106.426) (end 131.064 97.028) (width 0.5) (layer B.Cu) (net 2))
 (segment (start 131.064 97.028) (end 125.476 91.44) (width 0.5) (layer B.Cu) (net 2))
 (segment (start 125.476 91.44) (end 114.3 91.44) (width 0.5) (layer B.Cu) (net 2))
 (segment (start 114.3 91.44) (end 113.284 92.456) (width 0.5) (layer B.Cu) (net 2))
 (segment (start 113.284 94.996) (end 115.316 97.028) (width 0.5) (layer B.Cu) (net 2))
 (segment (start 113.284 92.456) (end 113.284 94.996) (width 0.5) (layer B.Cu) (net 2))
 (segment (start 94.742 109.22) (end 94.742 98.806) (width 0.5) (layer B.Cu) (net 17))
 (segment (start 94.742 98.806) (end 97.028 96.52) (width 0.5) (layer B.Cu) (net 17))
 (via (at 97.028 96.52) (size 0.8) (drill 0.4) (layers F.Cu B.Cu) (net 17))
 (segment (start 97.028 96.52) (end 100.076 93.472) (width 0.5) (layer F.Cu) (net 17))
 (via (at 100.076 93.472) (size 0.8) (drill 0.4) (layers F.Cu B.Cu) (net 17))
 (segment (start 100.076 93.472) (end 105.156 93.472) (width 0.5) (layer B.Cu) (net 17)))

